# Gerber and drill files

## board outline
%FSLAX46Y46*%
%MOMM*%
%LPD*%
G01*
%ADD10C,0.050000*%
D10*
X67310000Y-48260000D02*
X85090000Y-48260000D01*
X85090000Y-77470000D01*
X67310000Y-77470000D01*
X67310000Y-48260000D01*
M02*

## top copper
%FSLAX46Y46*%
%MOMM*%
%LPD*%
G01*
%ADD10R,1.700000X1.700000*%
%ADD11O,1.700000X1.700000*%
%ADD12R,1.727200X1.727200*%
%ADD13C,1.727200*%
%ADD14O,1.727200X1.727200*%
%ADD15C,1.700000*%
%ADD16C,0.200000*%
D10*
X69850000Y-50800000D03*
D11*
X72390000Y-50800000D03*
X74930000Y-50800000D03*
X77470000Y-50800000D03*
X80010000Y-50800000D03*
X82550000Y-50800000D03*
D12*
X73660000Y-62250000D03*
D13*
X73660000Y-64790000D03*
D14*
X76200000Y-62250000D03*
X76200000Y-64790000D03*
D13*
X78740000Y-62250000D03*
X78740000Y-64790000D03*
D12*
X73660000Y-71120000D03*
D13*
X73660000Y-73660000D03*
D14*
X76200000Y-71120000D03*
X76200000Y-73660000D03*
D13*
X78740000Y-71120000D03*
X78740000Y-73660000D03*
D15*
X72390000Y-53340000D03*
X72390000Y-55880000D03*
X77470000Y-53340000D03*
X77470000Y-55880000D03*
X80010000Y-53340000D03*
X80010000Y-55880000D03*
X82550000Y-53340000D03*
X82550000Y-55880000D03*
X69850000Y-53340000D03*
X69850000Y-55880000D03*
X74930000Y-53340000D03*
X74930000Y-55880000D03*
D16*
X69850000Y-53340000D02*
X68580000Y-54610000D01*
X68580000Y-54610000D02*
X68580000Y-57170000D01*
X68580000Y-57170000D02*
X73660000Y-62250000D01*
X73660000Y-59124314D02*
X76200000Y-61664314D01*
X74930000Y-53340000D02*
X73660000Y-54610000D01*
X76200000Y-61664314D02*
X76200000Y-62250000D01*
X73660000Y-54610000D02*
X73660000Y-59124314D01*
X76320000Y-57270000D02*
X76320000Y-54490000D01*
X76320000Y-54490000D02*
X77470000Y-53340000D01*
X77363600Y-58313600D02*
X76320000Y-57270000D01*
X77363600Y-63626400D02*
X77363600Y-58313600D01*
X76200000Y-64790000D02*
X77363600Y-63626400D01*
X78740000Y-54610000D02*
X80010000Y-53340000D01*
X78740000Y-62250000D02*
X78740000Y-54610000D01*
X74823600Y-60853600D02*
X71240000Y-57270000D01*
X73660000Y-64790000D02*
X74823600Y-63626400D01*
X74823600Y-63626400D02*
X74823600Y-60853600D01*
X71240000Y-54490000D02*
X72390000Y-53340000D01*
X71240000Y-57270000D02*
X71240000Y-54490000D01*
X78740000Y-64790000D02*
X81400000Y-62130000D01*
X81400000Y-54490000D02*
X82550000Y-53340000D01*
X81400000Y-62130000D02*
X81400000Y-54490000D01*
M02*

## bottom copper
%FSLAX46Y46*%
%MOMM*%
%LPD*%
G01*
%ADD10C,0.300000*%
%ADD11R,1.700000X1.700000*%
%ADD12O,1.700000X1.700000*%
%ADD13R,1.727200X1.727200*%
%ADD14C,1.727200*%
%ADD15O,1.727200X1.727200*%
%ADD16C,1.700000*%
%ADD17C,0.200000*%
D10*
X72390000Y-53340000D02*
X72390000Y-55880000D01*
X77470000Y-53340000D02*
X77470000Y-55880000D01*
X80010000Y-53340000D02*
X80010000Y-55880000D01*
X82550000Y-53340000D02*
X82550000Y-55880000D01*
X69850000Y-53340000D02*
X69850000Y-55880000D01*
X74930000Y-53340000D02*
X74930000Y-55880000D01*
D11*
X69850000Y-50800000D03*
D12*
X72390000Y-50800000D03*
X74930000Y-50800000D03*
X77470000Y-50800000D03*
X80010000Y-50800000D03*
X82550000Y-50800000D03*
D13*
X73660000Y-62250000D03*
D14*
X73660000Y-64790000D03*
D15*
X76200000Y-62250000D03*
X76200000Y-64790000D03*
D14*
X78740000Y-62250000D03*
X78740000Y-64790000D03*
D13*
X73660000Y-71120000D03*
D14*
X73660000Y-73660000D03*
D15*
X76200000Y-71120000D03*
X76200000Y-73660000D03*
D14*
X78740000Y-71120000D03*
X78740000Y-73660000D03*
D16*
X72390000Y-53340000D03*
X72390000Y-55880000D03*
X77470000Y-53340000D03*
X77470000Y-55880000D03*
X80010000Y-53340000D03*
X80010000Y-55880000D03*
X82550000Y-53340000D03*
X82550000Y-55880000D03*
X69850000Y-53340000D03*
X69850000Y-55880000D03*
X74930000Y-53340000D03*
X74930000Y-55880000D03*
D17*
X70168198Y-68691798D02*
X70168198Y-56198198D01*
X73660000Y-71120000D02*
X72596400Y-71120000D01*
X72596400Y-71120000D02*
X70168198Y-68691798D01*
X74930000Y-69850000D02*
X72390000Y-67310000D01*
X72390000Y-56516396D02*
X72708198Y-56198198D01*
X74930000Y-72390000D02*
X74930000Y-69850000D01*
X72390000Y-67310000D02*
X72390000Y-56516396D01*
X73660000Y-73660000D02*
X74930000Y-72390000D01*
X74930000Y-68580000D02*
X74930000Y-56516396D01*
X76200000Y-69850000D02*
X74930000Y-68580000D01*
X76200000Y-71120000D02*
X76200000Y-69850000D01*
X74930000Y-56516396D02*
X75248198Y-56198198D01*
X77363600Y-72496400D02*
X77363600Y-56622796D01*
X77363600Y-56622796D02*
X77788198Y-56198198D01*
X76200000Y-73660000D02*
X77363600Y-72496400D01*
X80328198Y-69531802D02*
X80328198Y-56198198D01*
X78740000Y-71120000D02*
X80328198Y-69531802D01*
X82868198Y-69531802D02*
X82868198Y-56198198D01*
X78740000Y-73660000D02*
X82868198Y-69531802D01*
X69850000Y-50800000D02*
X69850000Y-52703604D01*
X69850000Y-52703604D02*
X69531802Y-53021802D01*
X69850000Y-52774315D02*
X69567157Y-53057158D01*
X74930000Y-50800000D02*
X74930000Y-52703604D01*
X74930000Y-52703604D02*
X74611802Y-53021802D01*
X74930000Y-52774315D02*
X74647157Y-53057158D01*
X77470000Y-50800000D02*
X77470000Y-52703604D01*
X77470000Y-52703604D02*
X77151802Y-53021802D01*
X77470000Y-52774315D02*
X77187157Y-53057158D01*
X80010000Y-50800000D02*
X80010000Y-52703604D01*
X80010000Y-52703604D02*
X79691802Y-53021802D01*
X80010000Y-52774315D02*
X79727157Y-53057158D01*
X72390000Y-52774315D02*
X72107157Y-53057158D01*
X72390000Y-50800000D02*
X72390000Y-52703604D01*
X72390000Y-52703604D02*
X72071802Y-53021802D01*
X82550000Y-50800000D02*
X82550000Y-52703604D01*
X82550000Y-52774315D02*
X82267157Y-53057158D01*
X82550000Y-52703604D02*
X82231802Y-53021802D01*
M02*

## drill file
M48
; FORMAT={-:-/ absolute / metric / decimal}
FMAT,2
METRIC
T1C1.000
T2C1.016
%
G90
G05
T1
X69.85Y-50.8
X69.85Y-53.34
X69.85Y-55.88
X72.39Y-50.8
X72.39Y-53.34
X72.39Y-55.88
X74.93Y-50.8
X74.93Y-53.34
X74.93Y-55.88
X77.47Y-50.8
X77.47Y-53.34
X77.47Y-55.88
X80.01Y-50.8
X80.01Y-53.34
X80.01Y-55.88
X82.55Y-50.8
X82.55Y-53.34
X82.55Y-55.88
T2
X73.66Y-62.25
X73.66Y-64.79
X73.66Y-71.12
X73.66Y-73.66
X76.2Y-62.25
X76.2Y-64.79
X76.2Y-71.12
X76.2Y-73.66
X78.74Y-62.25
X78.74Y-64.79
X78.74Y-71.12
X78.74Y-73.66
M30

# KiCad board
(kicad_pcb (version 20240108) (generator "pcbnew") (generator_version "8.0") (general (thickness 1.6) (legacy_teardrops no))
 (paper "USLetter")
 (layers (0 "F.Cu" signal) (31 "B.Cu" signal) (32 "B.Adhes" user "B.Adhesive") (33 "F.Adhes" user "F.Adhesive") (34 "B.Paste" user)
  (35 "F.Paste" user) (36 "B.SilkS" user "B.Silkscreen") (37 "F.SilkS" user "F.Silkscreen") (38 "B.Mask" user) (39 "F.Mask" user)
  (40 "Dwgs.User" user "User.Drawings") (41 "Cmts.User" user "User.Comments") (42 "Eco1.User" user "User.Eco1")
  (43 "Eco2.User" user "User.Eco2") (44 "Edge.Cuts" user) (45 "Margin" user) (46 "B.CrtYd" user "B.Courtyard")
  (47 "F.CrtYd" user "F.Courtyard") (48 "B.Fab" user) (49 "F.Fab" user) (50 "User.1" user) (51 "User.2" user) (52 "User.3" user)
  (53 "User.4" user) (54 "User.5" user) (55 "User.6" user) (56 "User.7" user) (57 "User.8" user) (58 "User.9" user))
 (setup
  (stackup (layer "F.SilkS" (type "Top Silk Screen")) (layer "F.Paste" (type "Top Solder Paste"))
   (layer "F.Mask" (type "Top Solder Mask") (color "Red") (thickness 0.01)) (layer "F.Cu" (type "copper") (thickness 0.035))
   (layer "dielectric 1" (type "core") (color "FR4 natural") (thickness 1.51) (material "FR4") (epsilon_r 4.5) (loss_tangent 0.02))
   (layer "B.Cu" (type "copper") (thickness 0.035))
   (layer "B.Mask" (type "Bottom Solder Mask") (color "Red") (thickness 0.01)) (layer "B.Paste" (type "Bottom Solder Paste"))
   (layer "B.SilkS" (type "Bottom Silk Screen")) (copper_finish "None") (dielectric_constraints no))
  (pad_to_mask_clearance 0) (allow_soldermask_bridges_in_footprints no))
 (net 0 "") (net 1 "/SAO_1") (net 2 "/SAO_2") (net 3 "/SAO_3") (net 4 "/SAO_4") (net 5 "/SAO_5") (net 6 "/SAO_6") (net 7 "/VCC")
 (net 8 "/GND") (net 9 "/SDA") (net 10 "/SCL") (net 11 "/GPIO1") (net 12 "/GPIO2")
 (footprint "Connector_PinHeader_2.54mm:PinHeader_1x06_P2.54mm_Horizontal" (layer "F.Cu") (at 69.85 50.8 90)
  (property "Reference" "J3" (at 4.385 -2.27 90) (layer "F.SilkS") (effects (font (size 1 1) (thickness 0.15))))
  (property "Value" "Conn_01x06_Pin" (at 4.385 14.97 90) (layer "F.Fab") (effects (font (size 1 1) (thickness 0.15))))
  (pad "1" thru_hole rect (at 0 0 90) (size 1.7 1.7) (drill 1) (layers "*.Cu" "*.Mask") (remove_unused_layers no) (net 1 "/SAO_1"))
  (pad "2" thru_hole oval (at 0 2.54 90) (size 1.7 1.7) (drill 1) (layers "*.Cu" "*.Mask") (remove_unused_layers no) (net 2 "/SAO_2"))
  (pad "3" thru_hole oval (at 0 5.08 90) (size 1.7 1.7) (drill 1) (layers "*.Cu" "*.Mask") (remove_unused_layers no) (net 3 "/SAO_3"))
  (pad "4" thru_hole oval (at 0 7.62 90) (size 1.7 1.7) (drill 1) (layers "*.Cu" "*.Mask") (remove_unused_layers no) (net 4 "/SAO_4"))
  (pad "5" thru_hole oval (at 0 10.16 90) (size 1.7 1.7) (drill 1) (layers "*.Cu" "*.Mask") (remove_unused_layers no) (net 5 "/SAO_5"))
  (pad "6" thru_hole oval (at 0 12.7 90) (size 1.7 1.7) (drill 1) (layers "*.Cu" "*.Mask") (remove_unused_layers no) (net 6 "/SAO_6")))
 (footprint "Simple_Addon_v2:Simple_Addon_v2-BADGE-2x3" (layer "F.Cu") (at 76.14 63.5)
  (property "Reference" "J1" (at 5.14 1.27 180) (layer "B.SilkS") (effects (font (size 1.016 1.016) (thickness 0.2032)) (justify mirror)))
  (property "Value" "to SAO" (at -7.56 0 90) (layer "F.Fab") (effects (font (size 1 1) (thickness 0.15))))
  (pad "1" thru_hole rect (at -2.48 -1.25 270) (size 1.7272 1.7272) (drill 1.016) (layers "*.Cu" "*.Mask") (remove_unused_layers no)
   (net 1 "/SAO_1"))
  (pad "2" thru_hole circle (at -2.48 1.29 270) (size 1.7272 1.7272) (drill 1.016) (layers "*.Cu" "*.Mask") (remove_unused_layers no)
   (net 2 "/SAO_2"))
  (pad "3" thru_hole oval (at 0.06 -1.25 270) (size 1.7272 1.7272) (drill 1.016) (layers "*.Cu" "*.Mask") (remove_unused_layers no)
   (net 3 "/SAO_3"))
  (pad "4" thru_hole oval (at 0.06 1.29 270) (size 1.7272 1.7272) (drill 1.016) (layers "*.Cu" "*.Mask") (remove_unused_layers no)
   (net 4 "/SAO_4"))
  (pad "5" thru_hole circle (at 2.6 -1.25 270) (size 1.7272 1.7272) (drill 1.016) (layers "*.Cu" "*.Mask") (remove_unused_layers no)
   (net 5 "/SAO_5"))
  (pad "6" thru_hole circle (at 2.6 1.29 270) (size 1.7272 1.7272) (drill 1.016) (layers "*.Cu" "*.Mask") (remove_unused_layers no)
   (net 6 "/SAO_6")))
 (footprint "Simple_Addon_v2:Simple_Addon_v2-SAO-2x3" (layer "F.Cu") (at 76.14 72.37)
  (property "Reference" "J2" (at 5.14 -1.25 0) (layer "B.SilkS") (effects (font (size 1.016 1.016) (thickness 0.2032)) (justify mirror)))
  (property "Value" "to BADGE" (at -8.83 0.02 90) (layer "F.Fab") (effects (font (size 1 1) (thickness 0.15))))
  (pad "1" thru_hole rect (at -2.48 -1.25 270) (size 1.7272 1.7272) (drill 1.016) (layers "*.Cu" "*.Mask") (remove_unused_layers no)
   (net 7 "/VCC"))
  (pad "2" thru_hole circle (at -2.48 1.29 270) (size 1.7272 1.7272) (drill 1.016) (layers "*.Cu" "*.Mask") (remove_unused_layers no)
   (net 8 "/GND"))
  (pad "3" thru_hole oval (at 0.06 -1.25 270) (size 1.7272 1.7272) (drill 1.016) (layers "*.Cu" "*.Mask") (remove_unused_layers no)
   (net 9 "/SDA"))
  (pad "4" thru_hole oval (at 0.06 1.29 270) (size 1.7272 1.7272) (drill 1.016) (layers "*.Cu" "*.Mask") (remove_unused_layers no)
   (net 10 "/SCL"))
  (pad "5" thru_hole circle (at 2.6 -1.25 270) (size 1.7272 1.7272) (drill 1.016) (layers "*.Cu" "*.Mask") (remove_unused_layers no)
   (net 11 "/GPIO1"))
  (pad "6" thru_hole circle (at 2.6 1.29 270) (size 1.7272 1.7272) (drill 1.016) (layers "*.Cu" "*.Mask") (remove_unused_layers no)
   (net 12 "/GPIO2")))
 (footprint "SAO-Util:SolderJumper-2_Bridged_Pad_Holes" (layer "B.Cu") (at 72.39 53.34 -90)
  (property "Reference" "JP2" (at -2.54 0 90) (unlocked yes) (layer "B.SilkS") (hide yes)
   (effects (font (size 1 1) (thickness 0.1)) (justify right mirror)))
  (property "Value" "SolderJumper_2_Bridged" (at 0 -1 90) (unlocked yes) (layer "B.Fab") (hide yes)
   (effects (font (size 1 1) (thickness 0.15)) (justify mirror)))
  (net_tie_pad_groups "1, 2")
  (fp_line (start 0 0) (end 2.54 0) (stroke (width 0.3) (type default)) (layer "B.Cu"))
  (pad "1" thru_hole circle (at 0 0 270) (size 1.7 1.7) (drill 1) (layers "*.Cu" "*.Mask") (remove_unused_layers no) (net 2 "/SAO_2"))
  (pad "2" thru_hole circle (at 2.54 0 270) (size 1.7 1.7) (drill 1) (layers "*.Cu" "*.Mask") (remove_unused_layers no) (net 8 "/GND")))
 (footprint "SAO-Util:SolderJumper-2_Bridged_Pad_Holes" (layer "B.Cu") (at 77.47 53.34 -90)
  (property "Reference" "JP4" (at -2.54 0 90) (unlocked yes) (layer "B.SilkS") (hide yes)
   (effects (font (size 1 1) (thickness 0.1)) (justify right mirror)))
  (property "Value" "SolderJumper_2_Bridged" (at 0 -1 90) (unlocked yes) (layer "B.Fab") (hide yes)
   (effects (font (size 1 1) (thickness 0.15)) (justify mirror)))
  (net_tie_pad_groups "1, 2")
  (fp_line (start 0 0) (end 2.54 0) (stroke (width 0.3) (type default)) (layer "B.Cu"))
  (pad "1" thru_hole circle (at 0 0 270) (size 1.7 1.7) (drill 1) (layers "*.Cu" "*.Mask") (remove_unused_layers no) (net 4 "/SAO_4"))
  (pad "2" thru_hole circle (at 2.54 0 270) (size 1.7 1.7) (drill 1) (layers "*.Cu" "*.Mask") (remove_unused_layers no) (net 10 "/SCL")))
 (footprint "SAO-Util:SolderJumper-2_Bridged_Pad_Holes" (layer "B.Cu") (at 80.01 53.34 -90)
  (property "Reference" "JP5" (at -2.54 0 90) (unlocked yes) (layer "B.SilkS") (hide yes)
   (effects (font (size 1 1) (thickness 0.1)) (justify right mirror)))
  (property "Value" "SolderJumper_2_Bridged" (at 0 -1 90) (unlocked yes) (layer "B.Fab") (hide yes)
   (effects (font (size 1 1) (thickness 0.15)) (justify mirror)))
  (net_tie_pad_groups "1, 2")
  (fp_line (start 0 0) (end 2.54 0) (stroke (width 0.3) (type default)) (layer "B.Cu"))
  (pad "1" thru_hole circle (at 0 0 270) (size 1.7 1.7) (drill 1) (layers "*.Cu" "*.Mask") (remove_unused_layers no) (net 5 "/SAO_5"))
  (pad "2" thru_hole circle (at 2.54 0 270) (size 1.7 1.7) (drill 1) (layers "*.Cu" "*.Mask") (remove_unused_layers no) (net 11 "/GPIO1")))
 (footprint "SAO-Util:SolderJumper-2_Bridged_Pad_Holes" (layer "B.Cu") (at 82.55 53.34 -90)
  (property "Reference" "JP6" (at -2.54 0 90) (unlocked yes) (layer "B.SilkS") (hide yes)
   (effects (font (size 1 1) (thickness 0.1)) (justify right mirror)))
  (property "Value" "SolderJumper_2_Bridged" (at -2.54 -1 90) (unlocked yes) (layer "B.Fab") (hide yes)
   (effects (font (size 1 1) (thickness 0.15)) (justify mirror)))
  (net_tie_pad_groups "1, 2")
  (fp_line (start 0 0) (end 2.54 0) (stroke (width 0.3) (type default)) (layer "B.Cu"))
  (pad "1" thru_hole circle (at 0 0 270) (size 1.7 1.7) (drill 1) (layers "*.Cu" "*.Mask") (remove_unused_layers no) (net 6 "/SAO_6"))
  (pad "2" thru_hole circle (at 2.54 0 270) (size 1.7 1.7) (drill 1) (layers "*.Cu" "*.Mask") (remove_unused_layers no) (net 12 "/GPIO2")))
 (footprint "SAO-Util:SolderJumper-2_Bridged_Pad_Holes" (layer "B.Cu") (at 69.85 53.34 -90)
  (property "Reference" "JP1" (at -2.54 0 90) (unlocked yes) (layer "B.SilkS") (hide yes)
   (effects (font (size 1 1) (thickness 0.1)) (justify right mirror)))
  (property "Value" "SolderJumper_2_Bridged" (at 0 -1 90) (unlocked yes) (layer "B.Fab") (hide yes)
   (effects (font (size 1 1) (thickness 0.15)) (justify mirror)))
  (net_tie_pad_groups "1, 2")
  (fp_line (start 0 0) (end 2.54 0) (stroke (width 0.3) (type default)) (layer "B.Cu"))
  (pad "1" thru_hole circle (at 0 0 270) (size 1.7 1.7) (drill 1) (layers "*.Cu" "*.Mask") (remove_unused_layers no) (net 1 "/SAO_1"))
  (pad "2" thru_hole circle (at 2.54 0 270) (size 1.7 1.7) (drill 1) (layers "*.Cu" "*.Mask") (remove_unused_layers no) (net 7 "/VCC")))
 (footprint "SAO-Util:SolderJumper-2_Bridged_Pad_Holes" (layer "B.Cu") (at 74.93 53.34 -90)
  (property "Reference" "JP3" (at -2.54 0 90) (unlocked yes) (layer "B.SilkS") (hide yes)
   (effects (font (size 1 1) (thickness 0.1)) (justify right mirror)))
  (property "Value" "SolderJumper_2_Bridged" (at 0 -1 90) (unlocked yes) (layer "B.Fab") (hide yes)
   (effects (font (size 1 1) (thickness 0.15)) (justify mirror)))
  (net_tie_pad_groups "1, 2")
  (fp_line (start 0 0) (end 2.54 0) (stroke (width 0.3) (type default)) (layer "B.Cu"))
  (pad "1" thru_hole circle (at 0 0 270) (size 1.7 1.7) (drill 1) (layers "*.Cu" "*.Mask") (remove_unused_layers no) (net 3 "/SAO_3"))
  (pad "2" thru_hole circle (at 2.54 0 270) (size 1.7 1.7) (drill 1) (layers "*.Cu" "*.Mask") (remove_unused_layers no) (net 9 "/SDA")))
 (gr_rect (start 67.31 48.26) (end 85.09 77.47) (stroke (width 0.05) (type default)) (fill none) (layer "Edge.Cuts"))
 (segment (start 70.168198 68.691798) (end 70.168198 56.198198) (width 0.2) (layer "B.Cu") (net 7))
 (segment (start 73.66 71.12) (end 72.5964 71.12) (width 0.2) (layer "B.Cu") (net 7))
 (segment (start 72.5964 71.12) (end 70.168198 68.691798) (width 0.2) (layer "B.Cu") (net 7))
 (segment (start 74.93 69.85) (end 72.39 67.31) (width 0.2) (layer "B.Cu") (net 8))
 (segment (start 72.39 56.516396) (end 72.708198 56.198198) (width 0.2) (layer "B.Cu") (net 8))
 (segment (start 74.93 72.39) (end 74.93 69.85) (width 0.2) (layer "B.Cu") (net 8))
 (segment (start 72.39 67.31) (end 72.39 56.516396) (width 0.2) (layer "B.Cu") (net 8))
 (segment (start 73.66 73.66) (end 74.93 72.39) (width 0.2) (layer "B.Cu") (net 8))
 (segment (start 74.93 68.58) (end 74.93 56.516396) (width 0.2) (layer "B.Cu") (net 9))
 (segment (start 76.2 69.85) (end 74.93 68.58) (width 0.2) (layer "B.Cu") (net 9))
 (segment (start 76.2 71.12) (end 76.2 69.85) (width 0.2) (layer "B.Cu") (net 9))
 (segment (start 74.93 56.516396) (end 75.248198 56.198198) (width 0.2) (layer "B.Cu") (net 9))
 (segment (start 77.3636 72.4964) (end 77.3636 56.622796) (width 0.2) (layer "B.Cu") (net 10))
 (segment (start 77.3636 56.622796) (end 77.788198 56.198198) (width 0.2) (layer "B.Cu") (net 10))
 (segment (start 76.2 73.66) (end 77.3636 72.4964) (width 0.2) (layer "B.Cu") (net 10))
 (segment (start 80.328198 69.531802) (end 80.328198 56.198198) (width 0.2) (layer "B.Cu") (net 11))
 (segment (start 78.74 71.12) (end 80.328198 69.531802) (width 0.2) (layer "B.Cu") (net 11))
 (segment (start 82.868198 69.531802) (end 82.868198 56.198198) (width 0.2) (layer "B.Cu") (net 12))
 (segment (start 78.74 73.66) (end 82.868198 69.531802) (width 0.2) (layer "B.Cu") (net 12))
 (segment (start 69.85 53.34) (end 68.58 54.61) (width 0.2) (layer "F.Cu") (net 1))
 (segment (start 68.58 54.61) (end 68.58 57.17) (width 0.2) (layer "F.Cu") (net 1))
 (segment (start 68.58 57.17) (end 73.66 62.25) (width 0.2) (layer "F.Cu") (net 1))
 (segment (start 69.85 50.8) (end 69.85 52.703604) (width 0.2) (layer "B.Cu") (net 1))
 (segment (start 69.85 52.703604) (end 69.531802 53.021802) (width 0.2) (layer "B.Cu") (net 1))
 (segment (start 69.85 52.774315) (end 69.567157 53.057158) (width 0.2) (layer "B.Cu") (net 1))
 (segment (start 73.66 59.124314) (end 76.2 61.664314) (width 0.2) (layer "F.Cu") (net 3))
 (segment (start 74.93 53.34) (end 73.66 54.61) (width 0.2) (layer "F.Cu") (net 3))
 (segment (start 76.2 61.664314) (end 76.2 62.25) (width 0.2) (layer "F.Cu") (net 3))
 (segment (start 73.66 54.61) (end 73.66 59.124314) (width 0.2) (layer "F.Cu") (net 3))
 (segment (start 74.93 50.8) (end 74.93 52.703604) (width 0.2) (layer "B.Cu") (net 3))
 (segment (start 74.93 52.703604) (end 74.611802 53.021802) (width 0.2) (layer "B.Cu") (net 3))
 (segment (start 74.93 52.774315) (end 74.647157 53.057158) (width 0.2) (layer "B.Cu") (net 3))
 (segment (start 76.32 57.27) (end 76.32 54.49) (width 0.2) (layer "F.Cu") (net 4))
 (segment (start 76.32 54.49) (end 77.47 53.34) (width 0.2) (layer "F.Cu") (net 4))
 (segment (start 77.3636 58.3136) (end 76.32 57.27) (width 0.2) (layer "F.Cu") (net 4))
 (segment (start 77.3636 63.6264) (end 77.3636 58.3136) (width 0.2) (layer "F.Cu") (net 4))
 (segment (start 76.2 64.79) (end 77.3636 63.6264) (width 0.2) (layer "F.Cu") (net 4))
 (segment (start 77.47 50.8) (end 77.47 52.703604) (width 0.2) (layer "B.Cu") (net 4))
 (segment (start 77.47 52.703604) (end 77.151802 53.021802) (width 0.2) (layer "B.Cu") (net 4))
 (segment (start 77.47 52.774315) (end 77.187157 53.057158) (width 0.2) (layer "B.Cu") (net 4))
 (segment (start 78.74 54.61) (end 80.01 53.34) (width 0.2) (layer "F.Cu") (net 5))
 (segment (start 78.74 62.25) (end 78.74 54.61) (width 0.2) (layer "F.Cu") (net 5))
 (segment (start 80.01 50.8) (end 80.01 52.703604) (width 0.2) (layer "B.Cu") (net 5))
 (segment (start 80.01 52.703604) (end 79.691802 53.021802) (width 0.2) (layer "B.Cu") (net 5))
 (segment (start 80.01 52.774315) (end 79.727157 53.057158) (width 0.2) (layer "B.Cu") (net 5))
 (segment (start 74.8236 60.8536) (end 71.24 57.27) (width 0.2) (layer "F.Cu") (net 2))
 (segment (start 73.66 64.79) (end 74.8236 63.6264) (width 0.2) (layer "F.Cu") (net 2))
 (segment (start 74.8236 63.6264) (end 74.8236 60.8536) (width 0.2) (layer "F.Cu") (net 2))
 (segment (start 71.24 54.49) (end 72.39 53.34) (width 0.2) (layer "F.Cu") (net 2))
 (segment (start 71.24 57.27) (end 71.24 54.49) (width 0.2) (layer "F.Cu") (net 2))
 (segment (start 72.39 52.774315) (end 72.107157 53.057158) (width 0.2) (layer "B.Cu") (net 2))
 (segment (start 72.39 50.8) (end 72.39 52.703604) (width 0.2) (layer "B.Cu") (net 2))
 (segment (start 72.39 52.703604) (end 72.071802 53.021802) (width 0.2) (layer "B.Cu") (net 2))
 (segment (start 78.74 64.79) (end 81.4 62.13) (width 0.2) (layer "F.Cu") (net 6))
 (segment (start 81.4 54.49) (end 82.55 53.34) (width 0.2) (layer "F.Cu") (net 6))
 (segment (start 81.4 62.13) (end 81.4 54.49) (width 0.2) (layer "F.Cu") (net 6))
 (segment (start 82.55 50.8) (end 82.55 52.703604) (width 0.2) (layer "B.Cu") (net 6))
 (segment (start 82.55 52.774315) (end 82.267157 53.057158) (width 0.2) (layer "B.Cu") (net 6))
 (segment (start 82.55 52.703604) (end 82.231802 53.021802) (width 0.2) (layer "B.Cu") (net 6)))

